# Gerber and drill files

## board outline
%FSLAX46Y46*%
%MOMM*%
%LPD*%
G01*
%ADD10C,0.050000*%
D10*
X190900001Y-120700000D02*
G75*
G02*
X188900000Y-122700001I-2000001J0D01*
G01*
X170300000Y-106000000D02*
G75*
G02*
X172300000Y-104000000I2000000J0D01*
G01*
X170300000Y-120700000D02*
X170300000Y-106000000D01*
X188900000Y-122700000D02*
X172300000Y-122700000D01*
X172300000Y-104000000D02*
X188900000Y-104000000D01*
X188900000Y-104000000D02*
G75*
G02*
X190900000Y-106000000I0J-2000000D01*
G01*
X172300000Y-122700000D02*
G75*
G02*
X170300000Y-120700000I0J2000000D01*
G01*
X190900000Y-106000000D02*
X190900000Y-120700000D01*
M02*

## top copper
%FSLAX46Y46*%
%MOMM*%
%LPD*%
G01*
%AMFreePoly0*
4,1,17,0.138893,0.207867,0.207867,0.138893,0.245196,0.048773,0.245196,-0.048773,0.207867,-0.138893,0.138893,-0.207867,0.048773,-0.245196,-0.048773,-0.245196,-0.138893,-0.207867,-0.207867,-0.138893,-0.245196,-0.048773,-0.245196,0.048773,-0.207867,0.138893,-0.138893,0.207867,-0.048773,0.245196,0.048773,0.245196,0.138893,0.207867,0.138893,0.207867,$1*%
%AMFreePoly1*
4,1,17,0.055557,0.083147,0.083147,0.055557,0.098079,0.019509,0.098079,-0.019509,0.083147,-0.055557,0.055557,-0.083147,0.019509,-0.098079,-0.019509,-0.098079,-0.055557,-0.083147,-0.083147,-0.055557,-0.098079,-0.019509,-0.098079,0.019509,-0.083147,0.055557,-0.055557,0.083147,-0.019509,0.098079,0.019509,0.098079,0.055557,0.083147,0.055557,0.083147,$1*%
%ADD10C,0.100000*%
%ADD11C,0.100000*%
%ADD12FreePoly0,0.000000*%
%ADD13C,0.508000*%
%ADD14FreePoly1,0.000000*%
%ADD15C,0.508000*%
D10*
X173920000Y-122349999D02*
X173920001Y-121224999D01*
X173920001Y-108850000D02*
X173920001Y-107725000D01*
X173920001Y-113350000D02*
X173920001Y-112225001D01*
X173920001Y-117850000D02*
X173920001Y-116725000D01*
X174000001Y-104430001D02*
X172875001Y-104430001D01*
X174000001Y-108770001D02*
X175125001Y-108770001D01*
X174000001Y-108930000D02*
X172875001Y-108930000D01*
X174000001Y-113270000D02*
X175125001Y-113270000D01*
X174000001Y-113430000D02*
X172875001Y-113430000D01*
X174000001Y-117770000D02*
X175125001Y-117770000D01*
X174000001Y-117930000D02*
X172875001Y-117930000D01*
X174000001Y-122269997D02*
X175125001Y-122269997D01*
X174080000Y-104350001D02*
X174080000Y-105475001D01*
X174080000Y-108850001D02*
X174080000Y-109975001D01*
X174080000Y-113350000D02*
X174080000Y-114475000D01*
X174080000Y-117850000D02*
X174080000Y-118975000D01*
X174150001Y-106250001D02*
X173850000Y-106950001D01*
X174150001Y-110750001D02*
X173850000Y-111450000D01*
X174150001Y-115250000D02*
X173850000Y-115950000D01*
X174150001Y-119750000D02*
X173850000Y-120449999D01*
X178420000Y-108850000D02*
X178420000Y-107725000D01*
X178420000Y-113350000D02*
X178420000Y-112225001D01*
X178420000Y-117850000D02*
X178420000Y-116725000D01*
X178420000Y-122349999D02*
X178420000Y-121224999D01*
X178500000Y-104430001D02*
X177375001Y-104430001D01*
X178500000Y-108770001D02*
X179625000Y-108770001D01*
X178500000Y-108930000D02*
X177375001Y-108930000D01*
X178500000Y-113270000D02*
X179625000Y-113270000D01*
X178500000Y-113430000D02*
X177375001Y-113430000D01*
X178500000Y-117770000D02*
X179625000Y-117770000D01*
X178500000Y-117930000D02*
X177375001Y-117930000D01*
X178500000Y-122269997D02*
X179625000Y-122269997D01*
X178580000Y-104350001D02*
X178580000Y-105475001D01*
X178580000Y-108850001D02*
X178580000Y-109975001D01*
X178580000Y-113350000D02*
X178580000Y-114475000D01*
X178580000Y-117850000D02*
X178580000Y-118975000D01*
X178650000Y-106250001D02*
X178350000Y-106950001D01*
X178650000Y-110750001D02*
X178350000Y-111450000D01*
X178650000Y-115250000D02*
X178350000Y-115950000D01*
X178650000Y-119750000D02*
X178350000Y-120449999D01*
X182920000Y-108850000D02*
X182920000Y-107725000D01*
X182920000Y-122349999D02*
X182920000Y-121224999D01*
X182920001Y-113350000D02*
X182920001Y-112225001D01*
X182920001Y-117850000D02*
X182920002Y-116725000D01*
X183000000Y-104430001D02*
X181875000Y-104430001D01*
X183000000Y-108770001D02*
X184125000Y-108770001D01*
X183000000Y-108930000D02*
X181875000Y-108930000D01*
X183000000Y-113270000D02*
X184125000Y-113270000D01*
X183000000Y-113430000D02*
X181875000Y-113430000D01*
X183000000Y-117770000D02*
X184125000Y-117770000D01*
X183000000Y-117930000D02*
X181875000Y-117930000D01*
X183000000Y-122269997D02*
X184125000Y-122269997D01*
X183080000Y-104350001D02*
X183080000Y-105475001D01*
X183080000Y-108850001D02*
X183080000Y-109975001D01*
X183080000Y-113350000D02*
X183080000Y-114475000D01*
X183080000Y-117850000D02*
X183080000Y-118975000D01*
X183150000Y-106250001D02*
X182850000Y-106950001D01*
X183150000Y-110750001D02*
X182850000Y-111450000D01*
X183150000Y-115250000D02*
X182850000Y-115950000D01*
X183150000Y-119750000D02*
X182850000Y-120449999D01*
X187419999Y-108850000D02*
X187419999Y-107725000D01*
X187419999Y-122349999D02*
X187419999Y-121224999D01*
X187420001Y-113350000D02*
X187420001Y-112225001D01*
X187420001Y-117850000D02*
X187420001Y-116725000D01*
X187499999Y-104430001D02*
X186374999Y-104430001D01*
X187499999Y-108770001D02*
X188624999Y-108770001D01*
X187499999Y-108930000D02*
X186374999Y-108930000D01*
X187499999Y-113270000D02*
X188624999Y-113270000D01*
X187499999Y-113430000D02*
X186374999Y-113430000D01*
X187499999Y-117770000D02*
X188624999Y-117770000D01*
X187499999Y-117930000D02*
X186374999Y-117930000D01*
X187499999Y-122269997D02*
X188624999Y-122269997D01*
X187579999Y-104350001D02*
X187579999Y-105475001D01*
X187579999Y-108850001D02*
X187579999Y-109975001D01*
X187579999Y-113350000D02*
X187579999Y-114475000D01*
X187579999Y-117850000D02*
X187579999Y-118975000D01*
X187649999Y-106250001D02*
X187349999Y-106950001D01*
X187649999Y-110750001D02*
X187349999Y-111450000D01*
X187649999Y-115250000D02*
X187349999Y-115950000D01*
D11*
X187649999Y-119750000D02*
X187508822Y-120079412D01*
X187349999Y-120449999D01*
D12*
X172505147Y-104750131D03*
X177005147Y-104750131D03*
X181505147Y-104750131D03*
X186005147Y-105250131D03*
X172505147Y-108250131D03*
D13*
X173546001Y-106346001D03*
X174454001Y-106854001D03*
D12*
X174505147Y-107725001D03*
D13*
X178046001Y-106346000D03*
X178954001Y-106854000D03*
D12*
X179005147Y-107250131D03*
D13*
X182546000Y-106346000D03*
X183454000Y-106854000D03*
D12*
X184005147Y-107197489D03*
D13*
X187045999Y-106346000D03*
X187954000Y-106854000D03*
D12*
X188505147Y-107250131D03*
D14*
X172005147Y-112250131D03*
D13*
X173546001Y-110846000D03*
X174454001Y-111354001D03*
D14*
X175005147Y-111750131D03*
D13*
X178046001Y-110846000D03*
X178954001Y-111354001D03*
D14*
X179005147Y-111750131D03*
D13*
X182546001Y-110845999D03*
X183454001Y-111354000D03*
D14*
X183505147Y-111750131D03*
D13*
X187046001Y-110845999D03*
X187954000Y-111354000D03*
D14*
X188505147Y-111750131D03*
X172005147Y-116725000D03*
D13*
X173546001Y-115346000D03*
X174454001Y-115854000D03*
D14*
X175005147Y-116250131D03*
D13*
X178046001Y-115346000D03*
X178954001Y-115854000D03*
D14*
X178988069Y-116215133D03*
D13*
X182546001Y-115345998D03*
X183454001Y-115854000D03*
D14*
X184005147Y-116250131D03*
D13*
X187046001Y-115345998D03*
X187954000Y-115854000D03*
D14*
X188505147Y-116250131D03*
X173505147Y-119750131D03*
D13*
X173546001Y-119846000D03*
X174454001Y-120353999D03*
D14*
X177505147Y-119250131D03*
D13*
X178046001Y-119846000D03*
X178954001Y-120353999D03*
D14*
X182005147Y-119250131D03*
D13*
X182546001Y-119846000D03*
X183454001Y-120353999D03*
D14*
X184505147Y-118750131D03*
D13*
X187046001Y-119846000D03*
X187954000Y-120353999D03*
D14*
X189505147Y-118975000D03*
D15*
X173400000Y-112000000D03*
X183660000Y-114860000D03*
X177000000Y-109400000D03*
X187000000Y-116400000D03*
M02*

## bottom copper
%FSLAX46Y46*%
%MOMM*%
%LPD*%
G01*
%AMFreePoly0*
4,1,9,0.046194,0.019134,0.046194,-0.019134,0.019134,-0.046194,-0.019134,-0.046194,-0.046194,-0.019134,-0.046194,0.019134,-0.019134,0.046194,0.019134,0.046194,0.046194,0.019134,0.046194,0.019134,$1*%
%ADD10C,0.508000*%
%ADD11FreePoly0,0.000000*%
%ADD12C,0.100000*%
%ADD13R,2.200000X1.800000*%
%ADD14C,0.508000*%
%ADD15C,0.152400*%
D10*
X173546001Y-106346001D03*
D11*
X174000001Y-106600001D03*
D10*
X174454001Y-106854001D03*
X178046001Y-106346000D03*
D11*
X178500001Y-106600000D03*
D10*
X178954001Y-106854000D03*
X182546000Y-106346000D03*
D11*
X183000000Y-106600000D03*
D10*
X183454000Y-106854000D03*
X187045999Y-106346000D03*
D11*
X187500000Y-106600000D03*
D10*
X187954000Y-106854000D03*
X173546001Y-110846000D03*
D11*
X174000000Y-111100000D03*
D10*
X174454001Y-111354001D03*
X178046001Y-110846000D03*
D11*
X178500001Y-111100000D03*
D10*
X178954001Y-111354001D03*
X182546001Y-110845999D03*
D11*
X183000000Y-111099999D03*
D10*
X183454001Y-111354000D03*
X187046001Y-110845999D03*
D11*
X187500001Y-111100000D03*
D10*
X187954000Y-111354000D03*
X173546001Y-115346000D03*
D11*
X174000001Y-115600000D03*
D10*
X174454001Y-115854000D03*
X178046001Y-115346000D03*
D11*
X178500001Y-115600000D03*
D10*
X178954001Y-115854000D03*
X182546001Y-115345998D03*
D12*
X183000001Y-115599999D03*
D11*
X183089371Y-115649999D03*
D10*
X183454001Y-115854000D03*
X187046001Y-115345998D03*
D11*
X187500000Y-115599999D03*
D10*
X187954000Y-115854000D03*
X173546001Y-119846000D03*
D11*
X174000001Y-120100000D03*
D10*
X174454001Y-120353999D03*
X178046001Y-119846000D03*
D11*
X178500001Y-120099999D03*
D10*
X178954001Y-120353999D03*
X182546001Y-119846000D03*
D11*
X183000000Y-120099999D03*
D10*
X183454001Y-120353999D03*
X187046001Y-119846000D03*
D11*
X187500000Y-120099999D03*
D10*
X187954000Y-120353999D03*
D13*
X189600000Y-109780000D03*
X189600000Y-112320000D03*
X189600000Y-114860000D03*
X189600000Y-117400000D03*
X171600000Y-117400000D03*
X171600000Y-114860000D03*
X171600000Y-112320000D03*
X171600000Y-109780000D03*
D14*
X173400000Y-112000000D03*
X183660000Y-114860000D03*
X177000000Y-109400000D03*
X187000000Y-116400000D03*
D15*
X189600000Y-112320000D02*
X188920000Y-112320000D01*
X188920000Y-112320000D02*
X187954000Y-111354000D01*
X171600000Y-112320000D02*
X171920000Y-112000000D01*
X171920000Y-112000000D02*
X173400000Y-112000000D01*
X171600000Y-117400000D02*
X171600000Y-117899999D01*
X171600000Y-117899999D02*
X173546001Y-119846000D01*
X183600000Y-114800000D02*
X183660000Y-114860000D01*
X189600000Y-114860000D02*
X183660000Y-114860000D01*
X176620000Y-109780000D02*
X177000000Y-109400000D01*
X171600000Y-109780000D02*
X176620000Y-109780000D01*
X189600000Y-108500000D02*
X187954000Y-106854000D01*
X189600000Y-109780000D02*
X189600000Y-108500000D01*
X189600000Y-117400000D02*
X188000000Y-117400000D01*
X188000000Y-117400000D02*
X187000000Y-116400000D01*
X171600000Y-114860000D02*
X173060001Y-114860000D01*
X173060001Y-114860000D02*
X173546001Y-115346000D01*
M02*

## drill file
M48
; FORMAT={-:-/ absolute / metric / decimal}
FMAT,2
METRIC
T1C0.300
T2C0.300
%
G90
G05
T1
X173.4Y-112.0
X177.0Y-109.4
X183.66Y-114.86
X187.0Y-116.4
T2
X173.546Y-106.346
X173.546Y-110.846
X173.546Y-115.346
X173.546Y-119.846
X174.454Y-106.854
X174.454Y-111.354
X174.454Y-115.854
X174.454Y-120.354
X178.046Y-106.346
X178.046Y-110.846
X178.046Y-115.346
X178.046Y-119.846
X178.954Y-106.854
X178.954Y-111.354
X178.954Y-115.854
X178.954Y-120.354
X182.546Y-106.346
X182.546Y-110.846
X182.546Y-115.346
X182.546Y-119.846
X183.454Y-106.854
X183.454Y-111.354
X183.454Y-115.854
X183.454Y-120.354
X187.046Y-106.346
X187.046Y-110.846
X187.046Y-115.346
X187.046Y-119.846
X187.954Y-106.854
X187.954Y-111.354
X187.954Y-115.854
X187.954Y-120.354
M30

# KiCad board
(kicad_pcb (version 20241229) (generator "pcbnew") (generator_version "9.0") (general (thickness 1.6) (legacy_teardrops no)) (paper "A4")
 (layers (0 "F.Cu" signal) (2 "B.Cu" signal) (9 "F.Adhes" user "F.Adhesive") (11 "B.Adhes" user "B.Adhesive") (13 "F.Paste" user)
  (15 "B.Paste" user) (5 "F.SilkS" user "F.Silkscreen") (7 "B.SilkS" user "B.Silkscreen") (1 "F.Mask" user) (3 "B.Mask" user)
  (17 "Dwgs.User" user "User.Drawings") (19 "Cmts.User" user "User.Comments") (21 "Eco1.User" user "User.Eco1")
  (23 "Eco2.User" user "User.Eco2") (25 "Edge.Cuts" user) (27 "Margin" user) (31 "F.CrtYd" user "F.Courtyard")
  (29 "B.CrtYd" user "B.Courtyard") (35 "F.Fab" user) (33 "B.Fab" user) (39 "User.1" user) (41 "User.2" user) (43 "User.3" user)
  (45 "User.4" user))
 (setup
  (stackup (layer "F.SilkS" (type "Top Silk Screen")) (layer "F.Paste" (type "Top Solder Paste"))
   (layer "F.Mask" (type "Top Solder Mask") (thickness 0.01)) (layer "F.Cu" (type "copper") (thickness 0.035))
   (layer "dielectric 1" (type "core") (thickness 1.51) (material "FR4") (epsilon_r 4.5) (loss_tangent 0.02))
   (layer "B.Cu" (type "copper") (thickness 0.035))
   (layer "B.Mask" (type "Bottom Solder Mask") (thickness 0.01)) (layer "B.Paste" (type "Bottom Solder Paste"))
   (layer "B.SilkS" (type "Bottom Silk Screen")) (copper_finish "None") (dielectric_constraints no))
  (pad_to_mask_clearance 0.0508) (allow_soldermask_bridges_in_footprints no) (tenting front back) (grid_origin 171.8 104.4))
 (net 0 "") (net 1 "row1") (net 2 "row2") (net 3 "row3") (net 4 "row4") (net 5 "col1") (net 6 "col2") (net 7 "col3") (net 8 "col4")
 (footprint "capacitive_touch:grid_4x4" (layer "F.Cu") (at 180.505147 124.750131)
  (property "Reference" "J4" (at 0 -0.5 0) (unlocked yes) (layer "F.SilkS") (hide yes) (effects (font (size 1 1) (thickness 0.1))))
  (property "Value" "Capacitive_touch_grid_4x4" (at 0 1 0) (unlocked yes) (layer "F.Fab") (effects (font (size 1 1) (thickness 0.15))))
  (fp_line (start -6.585147 -2.400132) (end -6.585146 -3.525132) (stroke (width 0.1) (type solid)) (layer "F.Cu"))
  (fp_line (start -6.585146 -15.900131) (end -6.585146 -17.025131) (stroke (width 0.1) (type solid)) (layer "F.Cu"))
  (fp_line (start -6.585146 -11.400131) (end -6.585146 -12.52513) (stroke (width 0.1) (type solid)) (layer "F.Cu"))
  (fp_line (start -6.585146 -6.900131) (end -6.585146 -8.025131) (stroke (width 0.1) (type solid)) (layer "F.Cu"))
  (fp_line (start -6.505146 -20.32013) (end -7.630146 -20.32013) (stroke (width 0.1) (type solid)) (layer "F.Cu"))
  (fp_line (start -6.505146 -15.98013) (end -5.380146 -15.98013) (stroke (width 0.1) (type solid)) (layer "F.Cu"))
  (fp_line (start -6.505146 -15.820131) (end -7.630146 -15.820131) (stroke (width 0.1) (type solid)) (layer "F.Cu"))
  (fp_line (start -6.505146 -11.480131) (end -5.380146 -11.480131) (stroke (width 0.1) (type solid)) (layer "F.Cu"))
  (fp_line (start -6.505146 -11.320131) (end -7.630146 -11.320131) (stroke (width 0.1) (type solid)) (layer "F.Cu"))
  (fp_line (start -6.505146 -6.980131) (end -5.380146 -6.980131) (stroke (width 0.1) (type solid)) (layer "F.Cu"))
  (fp_line (start -6.505146 -6.820131) (end -7.630146 -6.820131) (stroke (width 0.1) (type solid)) (layer "F.Cu"))
  (fp_line (start -6.505146 -2.480134) (end -5.380146 -2.480134) (stroke (width 0.1) (type solid)) (layer "F.Cu"))
  (fp_line (start -6.425147 -20.40013) (end -6.425147 -19.27513) (stroke (width 0.1) (type solid)) (layer "F.Cu"))
  (fp_line (start -6.425147 -15.90013) (end -6.425147 -14.77513) (stroke (width 0.1) (type solid)) (layer "F.Cu"))
  (fp_line (start -6.425147 -11.400131) (end -6.425147 -10.275131) (stroke (width 0.1) (type solid)) (layer "F.Cu"))
  (fp_line (start -6.425147 -6.900131) (end -6.425147 -5.775131) (stroke (width 0.1) (type solid)) (layer "F.Cu"))
  (fp_line (start -6.355146 -18.50013) (end -6.655147 -17.80013) (stroke (width 0.1) (type solid)) (layer "F.Cu"))
  (fp_line (start -6.355146 -14.00013) (end -6.655147 -13.300131) (stroke (width 0.1) (type solid)) (layer "F.Cu"))
  (fp_line (start -6.355146 -9.500131) (end -6.655147 -8.800131) (stroke (width 0.1) (type solid)) (layer "F.Cu"))
  (fp_line (start -6.355146 -5.000131) (end -6.655147 -4.300132) (stroke (width 0.1) (type solid)) (layer "F.Cu"))
  (fp_line (start -2.085147 -15.900131) (end -2.085147 -17.025131) (stroke (width 0.1) (type solid)) (layer "F.Cu"))
  (fp_line (start -2.085147 -11.400131) (end -2.085147 -12.52513) (stroke (width 0.1) (type solid)) (layer "F.Cu"))
  (fp_line (start -2.085147 -6.900131) (end -2.085147 -8.025131) (stroke (width 0.1) (type solid)) (layer "F.Cu"))
  (fp_line (start -2.085147 -2.400132) (end -2.085147 -3.525132) (stroke (width 0.1) (type solid)) (layer "F.Cu"))
  (fp_line (start -2.005147 -20.32013) (end -3.130146 -20.32013) (stroke (width 0.1) (type solid)) (layer "F.Cu"))
  (fp_line (start -2.005147 -15.98013) (end -0.880147 -15.98013) (stroke (width 0.1) (type solid)) (layer "F.Cu"))
  (fp_line (start -2.005147 -15.820131) (end -3.130146 -15.820131) (stroke (width 0.1) (type solid)) (layer "F.Cu"))
  (fp_line (start -2.005147 -11.480131) (end -0.880147 -11.480131) (stroke (width 0.1) (type solid)) (layer "F.Cu"))
  (fp_line (start -2.005147 -11.320131) (end -3.130146 -11.320131) (stroke (width 0.1) (type solid)) (layer "F.Cu"))
  (fp_line (start -2.005147 -6.980131) (end -0.880147 -6.980131) (stroke (width 0.1) (type solid)) (layer "F.Cu"))
  (fp_line (start -2.005147 -6.820131) (end -3.130146 -6.820131) (stroke (width 0.1) (type solid)) (layer "F.Cu"))
  (fp_line (start -2.005147 -2.480134) (end -0.880147 -2.480134) (stroke (width 0.1) (type solid)) (layer "F.Cu"))
  (fp_line (start -1.925147 -20.40013) (end -1.925147 -19.27513) (stroke (width 0.1) (type solid)) (layer "F.Cu"))
  (fp_line (start -1.925147 -15.90013) (end -1.925147 -14.77513) (stroke (width 0.1) (type solid)) (layer "F.Cu"))
  (fp_line (start -1.925147 -11.400131) (end -1.925147 -10.275131) (stroke (width 0.1) (type solid)) (layer "F.Cu"))
  (fp_line (start -1.925147 -6.900131) (end -1.925147 -5.775131) (stroke (width 0.1) (type solid)) (layer "F.Cu"))
  (fp_line (start -1.855147 -18.50013) (end -2.155147 -17.80013) (stroke (width 0.1) (type solid)) (layer "F.Cu"))
  (fp_line (start -1.855147 -14.00013) (end -2.155147 -13.300131) (stroke (width 0.1) (type solid)) (layer "F.Cu"))
  (fp_line (start -1.855147 -9.500131) (end -2.155147 -8.800131) (stroke (width 0.1) (type solid)) (layer "F.Cu"))
  (fp_line (start -1.855147 -5.000131) (end -2.155147 -4.300132) (stroke (width 0.1) (type solid)) (layer "F.Cu"))
  (fp_line (start 2.414853 -15.900131) (end 2.414853 -17.025131) (stroke (width 0.1) (type solid)) (layer "F.Cu"))
  (fp_line (start 2.414853 -2.400132) (end 2.414853 -3.525132) (stroke (width 0.1) (type solid)) (layer "F.Cu"))
  (fp_line (start 2.414854 -11.400131) (end 2.414854 -12.52513) (stroke (width 0.1) (type solid)) (layer "F.Cu"))
  (fp_line (start 2.414854 -6.900131) (end 2.414855 -8.025131) (stroke (width 0.1) (type solid)) (layer "F.Cu"))
  (fp_line (start 2.494853 -20.32013) (end 1.369853 -20.32013) (stroke (width 0.1) (type solid)) (layer "F.Cu"))
  (fp_line (start 2.494853 -15.98013) (end 3.619853 -15.98013) (stroke (width 0.1) (type solid)) (layer "F.Cu"))
  (fp_line (start 2.494853 -15.820131) (end 1.369853 -15.820131) (stroke (width 0.1) (type solid)) (layer "F.Cu"))
  (fp_line (start 2.494853 -11.480131) (end 3.619853 -11.480131) (stroke (width 0.1) (type solid)) (layer "F.Cu"))
  (fp_line (start 2.494853 -11.320131) (end 1.369853 -11.320131) (stroke (width 0.1) (type solid)) (layer "F.Cu"))
  (fp_line (start 2.494853 -6.980131) (end 3.619853 -6.980131) (stroke (width 0.1) (type solid)) (layer "F.Cu"))
  (fp_line (start 2.494853 -6.820131) (end 1.369853 -6.820131) (stroke (width 0.1) (type solid)) (layer "F.Cu"))
  (fp_line (start 2.494853 -2.480134) (end 3.619853 -2.480134) (stroke (width 0.1) (type solid)) (layer "F.Cu"))
  (fp_line (start 2.574853 -20.40013) (end 2.574853 -19.27513) (stroke (width 0.1) (type solid)) (layer "F.Cu"))
  (fp_line (start 2.574853 -15.90013) (end 2.574853 -14.77513) (stroke (width 0.1) (type solid)) (layer "F.Cu"))
  (fp_line (start 2.574853 -11.400131) (end 2.574853 -10.275131) (stroke (width 0.1) (type solid)) (layer "F.Cu"))
  (fp_line (start 2.574853 -6.900131) (end 2.574853 -5.775131) (stroke (width 0.1) (type solid)) (layer "F.Cu"))
  (fp_line (start 2.644853 -18.50013) (end 2.344853 -17.80013) (stroke (width 0.1) (type solid)) (layer "F.Cu"))
  (fp_line (start 2.644853 -14.00013) (end 2.344853 -13.300131) (stroke (width 0.1) (type solid)) (layer "F.Cu"))
  (fp_line (start 2.644853 -9.500131) (end 2.344853 -8.800131) (stroke (width 0.1) (type solid)) (layer "F.Cu"))
  (fp_line (start 2.644853 -5.000131) (end 2.344853 -4.300132) (stroke (width 0.1) (type solid)) (layer "F.Cu"))
  (fp_line (start 6.914852 -15.900131) (end 6.914852 -17.025131) (stroke (width 0.1) (type solid)) (layer "F.Cu"))
  (fp_line (start 6.914852 -2.400132) (end 6.914852 -3.525132) (stroke (width 0.1) (type solid)) (layer "F.Cu"))
  (fp_line (start 6.914854 -11.400131) (end 6.914854 -12.52513) (stroke (width 0.1) (type solid)) (layer "F.Cu"))
  (fp_line (start 6.914854 -6.900131) (end 6.914854 -8.025131) (stroke (width 0.1) (type solid)) (layer "F.Cu"))
  (fp_line (start 6.994852 -20.32013) (end 5.869852 -20.32013) (stroke (width 0.1) (type solid)) (layer "F.Cu"))
  (fp_line (start 6.994852 -15.98013) (end 8.119852 -15.98013) (stroke (width 0.1) (type solid)) (layer "F.Cu"))
  (fp_line (start 6.994852 -15.820131) (end 5.869852 -15.820131) (stroke (width 0.1) (type solid)) (layer "F.Cu"))
  (fp_line (start 6.994852 -11.480131) (end 8.119852 -11.480131) (stroke (width 0.1) (type solid)) (layer "F.Cu"))
  (fp_line (start 6.994852 -11.320131) (end 5.869852 -11.320131) (stroke (width 0.1) (type solid)) (layer "F.Cu"))
  (fp_line (start 6.994852 -6.980131) (end 8.119852 -6.980131) (stroke (width 0.1) (type solid)) (layer "F.Cu"))
  (fp_line (start 6.994852 -6.820131) (end 5.869852 -6.820131) (stroke (width 0.1) (type solid)) (layer "F.Cu"))
  (fp_line (start 6.994852 -2.480134) (end 8.119852 -2.480134) (stroke (width 0.1) (type solid)) (layer "F.Cu"))
  (fp_line (start 7.074852 -20.40013) (end 7.074852 -19.27513) (stroke (width 0.1) (type solid)) (layer "F.Cu"))
  (fp_line (start 7.074852 -15.90013) (end 7.074852 -14.77513) (stroke (width 0.1) (type solid)) (layer "F.Cu"))
  (fp_line (start 7.074852 -11.400131) (end 7.074852 -10.275131) (stroke (width 0.1) (type solid)) (layer "F.Cu"))
  (fp_line (start 7.074852 -6.900131) (end 7.074852 -5.775131) (stroke (width 0.1) (type solid)) (layer "F.Cu"))
  (fp_line (start 7.144852 -18.50013) (end 6.844852 -17.80013) (stroke (width 0.1) (type solid)) (layer "F.Cu"))
  (fp_line (start 7.144852 -14.00013) (end 6.844852 -13.300131) (stroke (width 0.1) (type solid)) (layer "F.Cu"))
  (fp_line (start 7.144852 -9.500131) (end 6.844852 -8.800131) (stroke (width 0.1) (type solid)) (layer "F.Cu"))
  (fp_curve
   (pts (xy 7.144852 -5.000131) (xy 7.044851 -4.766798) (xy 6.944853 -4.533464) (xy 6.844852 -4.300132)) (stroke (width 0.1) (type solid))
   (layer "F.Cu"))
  (pad "1" smd custom (at -8 -20) (size 0.5 0.5) (layers "F.Cu") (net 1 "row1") (options (clearance outline) (anchor circle)) (primitives))
  (pad "2" smd custom (at -3.5 -20) (size 0.5 0.5) (layers "F.Cu") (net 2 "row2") (options (clearance outline) (anchor circle)) (primitives))
  (pad "3" smd custom (at 1 -20) (size 0.5 0.5) (layers "F.Cu") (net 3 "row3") (options (clearance outline) (anchor circle)) (primitives))
  (pad "4" smd custom (at 5.5 -19.5) (size 0.5 0.5) (layers "F.Cu") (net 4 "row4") (options (clearance outline) (anchor circle))
   (primitives))
  (pad "5" smd custom (at -8 -16.5) (size 0.5 0.5) (layers "F.Cu") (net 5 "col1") (options (clearance outline) (anchor circle)) (primitives))
  (pad "5" thru_hole circle (at -6.959146 -18.40413) (size 0.508 0.508) (drill 0.3) (layers "*.Cu") (remove_unused_layers no) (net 5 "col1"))
  (pad "5" smd custom (at -6.505146 -18.15013) (size 0.1 0.1) (layers "B.Cu") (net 5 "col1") (options (clearance outline) (anchor circle))
   (primitives))
  (pad "5" thru_hole circle (at -6.051146 -17.89613) (size 0.508 0.508) (drill 0.3) (layers "*.Cu") (remove_unused_layers no) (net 5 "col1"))
  (pad "5" smd custom (at -6 -17.02513) (size 0.5 0.5) (layers "F.Cu") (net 5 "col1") (options (clearance outline) (anchor circle))
   (primitives))
  (pad "5" thru_hole circle (at -2.459146 -18.404131) (size 0.508 0.508) (drill 0.3) (layers "*.Cu") (remove_unused_layers no)
   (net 5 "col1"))
  (pad "5" smd custom (at -2.005146 -18.150131) (size 0.1 0.1) (layers "B.Cu") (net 5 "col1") (options (clearance outline) (anchor circle))
   (primitives))
  (pad "5" thru_hole circle (at -1.551146 -17.896131) (size 0.508 0.508) (drill 0.3) (layers "*.Cu") (remove_unused_layers no)
   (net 5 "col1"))
  (pad "5" smd custom (at -1.5 -17.5) (size 0.5 0.5) (layers "F.Cu") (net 5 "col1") (options (clearance outline) (anchor circle))
   (primitives))
  (pad "5" thru_hole circle (at 2.040853 -18.404131) (size 0.508 0.508) (drill 0.3) (layers "*.Cu") (remove_unused_layers no) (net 5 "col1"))
  (pad "5" smd custom (at 2.494853 -18.150131) (size 0.1 0.1) (layers "B.Cu") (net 5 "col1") (options (clearance outline) (anchor circle))
   (primitives))
  (pad "5" thru_hole circle (at 2.948853 -17.896131) (size 0.508 0.508) (drill 0.3) (layers "*.Cu") (remove_unused_layers no) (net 5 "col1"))
  (pad "5" smd custom (at 3.5 -17.552642) (size 0.5 0.5) (layers "F.Cu") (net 5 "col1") (options (clearance outline) (anchor circle))
   (primitives))
  (pad "5" thru_hole circle (at 6.540852 -18.404131) (size 0.508 0.508) (drill 0.3) (layers "*.Cu") (remove_unused_layers no) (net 5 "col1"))
  (pad "5" smd custom (at 6.994853 -18.150131) (size 0.1 0.1) (layers "B.Cu") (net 5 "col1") (options (clearance outline) (anchor circle))
   (primitives))
  (pad "5" thru_hole circle (at 7.448853 -17.896131) (size 0.508 0.508) (drill 0.3) (layers "*.Cu") (remove_unused_layers no) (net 5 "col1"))
  (pad "5" smd custom (at 8 -17.5) (size 0.5 0.5) (layers "F.Cu") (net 5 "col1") (options (clearance outline) (anchor circle)) (primitives))
  (pad "6" smd custom (at -8.5 -12.5) (size 0.2 0.2) (layers "F.Cu") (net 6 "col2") (options (clearance outline) (anchor circle))
   (primitives))
  (pad "6" thru_hole circle (at -6.959146 -13.904131) (size 0.508 0.508) (drill 0.3) (layers "*.Cu") (remove_unused_layers no)
   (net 6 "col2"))
  (pad "6" smd custom (at -6.505147 -13.650131) (size 0.1 0.1) (layers "B.Cu") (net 6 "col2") (options (clearance outline) (anchor circle))
   (primitives))
  (pad "6" thru_hole circle (at -6.051146 -13.39613) (size 0.508 0.508) (drill 0.3) (layers "*.Cu") (remove_unused_layers no) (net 6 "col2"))
  (pad "6" smd custom (at -5.5 -13) (size 0.2 0.2) (layers "F.Cu") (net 6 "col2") (options (clearance outline) (anchor circle)) (primitives))
  (pad "6" thru_hole circle (at -2.459146 -13.904131) (size 0.508 0.508) (drill 0.3) (layers "*.Cu") (remove_unused_layers no)
   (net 6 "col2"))
  (pad "6" smd custom (at -2.005146 -13.650131) (size 0.1 0.1) (layers "B.Cu") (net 6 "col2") (options (clearance outline) (anchor circle))
   (primitives))
  (pad "6" thru_hole circle (at -1.551146 -13.39613) (size 0.508 0.508) (drill 0.3) (layers "*.Cu") (remove_unused_layers no) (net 6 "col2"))
  (pad "6" smd custom (at -1.5 -13) (size 0.2 0.2) (layers "F.Cu") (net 6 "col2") (options (clearance outline) (anchor circle)) (primitives))
  (pad "6" thru_hole circle (at 2.040854 -13.904132) (size 0.508 0.508) (drill 0.3) (layers "*.Cu") (remove_unused_layers no) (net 6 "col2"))
  (pad "6" smd custom (at 2.494853 -13.650132) (size 0.1 0.1) (layers "B.Cu") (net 6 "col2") (options (clearance outline) (anchor circle))
   (primitives))
  (pad "6" thru_hole circle (at 2.948854 -13.396131) (size 0.508 0.508) (drill 0.3) (layers "*.Cu") (remove_unused_layers no) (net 6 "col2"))
  (pad "6" smd custom (at 3 -13) (size 0.2 0.2) (layers "F.Cu") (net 6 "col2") (options (clearance outline) (anchor circle)) (primitives))
  (pad "6" thru_hole circle (at 6.540854 -13.904132) (size 0.508 0.508) (drill 0.3) (layers "*.Cu") (remove_unused_layers no) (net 6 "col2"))
  (pad "6" smd custom (at 6.994854 -13.650131) (size 0.1 0.1) (layers "B.Cu") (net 6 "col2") (options (clearance outline) (anchor circle))
   (primitives))
  (pad "6" thru_hole circle (at 7.448853 -13.396131) (size 0.508 0.508) (drill 0.3) (layers "*.Cu") (remove_unused_layers no) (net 6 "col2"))
  (pad "6" smd custom (at 8 -13) (size 0.2 0.2) (layers "F.Cu") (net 6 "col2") (options (clearance outline) (anchor circle)) (primitives))
  (pad "7" smd custom (at -8.5 -8.025131) (size 0.2 0.2) (layers "F.Cu") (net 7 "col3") (options (clearance outline) (anchor circle))
   (primitives))
  (pad "7" thru_hole circle (at -6.959146 -9.404131) (size 0.508 0.508) (drill 0.3) (layers "*.Cu") (remove_unused_layers no) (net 7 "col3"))
  (pad "7" smd custom (at -6.505146 -9.150131) (size 0.1 0.1) (layers "B.Cu") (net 7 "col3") (options (clearance outline) (anchor circle))
   (primitives))
  (pad "7" thru_hole circle (at -6.051146 -8.896131) (size 0.508 0.508) (drill 0.3) (layers "*.Cu") (remove_unused_layers no) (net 7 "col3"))
  (pad "7" smd custom (at -5.5 -8.5) (size 0.2 0.2) (layers "F.Cu") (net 7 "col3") (options (clearance outline) (anchor circle))
   (primitives))
  (pad "7" thru_hole circle (at -2.459146 -9.404131) (size 0.508 0.508) (drill 0.3) (layers "*.Cu") (remove_unused_layers no) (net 7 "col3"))
  (pad "7" smd custom (at -2.005146 -9.150131) (size 0.1 0.1) (layers "B.Cu") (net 7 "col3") (options (clearance outline) (anchor circle))
   (primitives))
  (pad "7" thru_hole circle (at -1.551146 -8.896131) (size 0.508 0.508) (drill 0.3) (layers "*.Cu") (remove_unused_layers no) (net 7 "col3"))
  (pad "7" smd custom (at -1.517078 -8.534998) (size 0.2 0.2) (layers "F.Cu") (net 7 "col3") (options (clearance outline) (anchor circle))
   (primitives))
  (pad "7" thru_hole circle (at 2.040854 -9.404133) (size 0.508 0.508) (drill 0.3) (layers "*.Cu") (remove_unused_layers no) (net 7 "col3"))
  (pad "7" smd circle (at 2.494854 -9.150132) (size 0.1 0.1) (layers "B.Cu") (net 7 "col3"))
  (pad "7" smd custom (at 2.584224 -9.100132) (size 0.1 0.1) (layers "B.Cu") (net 7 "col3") (options (clearance outline) (anchor circle))
   (primitives))
  (pad "7" thru_hole circle (at 2.948854 -8.896131) (size 0.508 0.508) (drill 0.3) (layers "*.Cu") (remove_unused_layers no) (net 7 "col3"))
  (pad "7" smd custom (at 3.5 -8.5) (size 0.2 0.2) (layers "F.Cu") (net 7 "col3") (options (clearance outline) (anchor circle)) (primitives))
  (pad "7" thru_hole circle (at 6.540854 -9.404133) (size 0.508 0.508) (drill 0.3) (layers "*.Cu") (remove_unused_layers no) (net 7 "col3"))
  (pad "7" smd custom (at 6.994853 -9.150132) (size 0.1 0.1) (layers "B.Cu") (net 7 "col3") (options (clearance outline) (anchor circle))
   (primitives))
  (pad "7" thru_hole circle (at 7.448853 -8.896131) (size 0.508 0.508) (drill 0.3) (layers "*.Cu") (remove_unused_layers no) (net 7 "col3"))
  (pad "7" smd custom (at 8 -8.5) (size 0.2 0.2) (layers "F.Cu") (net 7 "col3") (options (clearance outline) (anchor circle)) (primitives))
  (pad "8" smd custom (at -7 -5) (size 0.2 0.2) (layers "F.Cu") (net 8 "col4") (options (clearance outline) (anchor circle)) (primitives))
  (pad "8" thru_hole circle (at -6.959146 -4.904131) (size 0.508 0.508) (drill 0.3) (layers "*.Cu") (remove_unused_layers no) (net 8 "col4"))
  (pad "8" smd custom (at -6.505146 -4.650131) (size 0.1 0.1) (layers "B.Cu") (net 8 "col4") (options (clearance outline) (anchor circle))
   (primitives))
  (pad "8" thru_hole circle (at -6.051146 -4.396132) (size 0.508 0.508) (drill 0.3) (layers "*.Cu") (remove_unused_layers no) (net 8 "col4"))
  (pad "8" smd custom (at -3 -5.5) (size 0.2 0.2) (layers "F.Cu") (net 8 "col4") (options (clearance outline) (anchor circle)) (primitives))
  (pad "8" thru_hole circle (at -2.459146 -4.904131) (size 0.508 0.508) (drill 0.3) (layers "*.Cu") (remove_unused_layers no) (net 8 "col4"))
  (pad "8" smd custom (at -2.005146 -4.650132) (size 0.1 0.1) (layers "B.Cu") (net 8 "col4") (options (clearance outline) (anchor circle))
   (primitives))
  (pad "8" thru_hole circle (at -1.551146 -4.396132) (size 0.508 0.508) (drill 0.3) (layers "*.Cu") (remove_unused_layers no) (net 8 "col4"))
  (pad "8" smd custom (at 1.5 -5.5) (size 0.2 0.2) (layers "F.Cu") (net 8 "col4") (options (clearance outline) (anchor circle)) (primitives))
  (pad "8" thru_hole circle (at 2.040854 -4.904131) (size 0.508 0.508) (drill 0.3) (layers "*.Cu") (remove_unused_layers no) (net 8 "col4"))
  (pad "8" smd custom (at 2.494853 -4.650132) (size 0.1 0.1) (layers "B.Cu") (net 8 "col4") (options (clearance outline) (anchor circle))
   (primitives))
  (pad "8" thru_hole circle (at 2.948854 -4.396132) (size 0.508 0.508) (drill 0.3) (layers "*.Cu") (remove_unused_layers no) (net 8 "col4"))
  (pad "8" smd custom (at 4 -6) (size 0.2 0.2) (layers "F.Cu") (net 8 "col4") (options (clearance outline) (anchor circle)) (primitives))
  (pad "8" thru_hole circle (at 6.540854 -4.904131) (size 0.508 0.508) (drill 0.3) (layers "*.Cu") (remove_unused_layers no) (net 8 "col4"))
  (pad "8" smd custom (at 6.994853 -4.650132) (size 0.1 0.1) (layers "B.Cu") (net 8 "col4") (options (clearance outline) (anchor circle))
   (primitives))
  (pad "8" thru_hole circle (at 7.448853 -4.396132) (size 0.508 0.508) (drill 0.3) (layers "*.Cu") (remove_unused_layers no) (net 8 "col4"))
  (pad "8" smd custom (at 9 -5.775131) (size 0.2 0.2) (layers "F.Cu") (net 8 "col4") (options (clearance outline) (anchor circle))
   (primitives)))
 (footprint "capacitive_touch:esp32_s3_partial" (layer "B.Cu") (at 180.6 113.59 -90)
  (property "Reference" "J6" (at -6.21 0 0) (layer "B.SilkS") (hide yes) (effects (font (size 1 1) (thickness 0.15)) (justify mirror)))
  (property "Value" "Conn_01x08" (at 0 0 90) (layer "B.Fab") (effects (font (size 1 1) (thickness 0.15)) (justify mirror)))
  (pad "1" smd rect (at -3.81 -9 270) (size 1.8 2.2) (layers "B.Cu" "B.Mask" "B.Paste") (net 5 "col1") (thermal_bridge_angle 45))
  (pad "2" smd rect (at -1.27 -9 270) (size 1.8 2.2) (layers "B.Cu" "B.Mask" "B.Paste") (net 6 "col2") (thermal_bridge_angle 45))
  (pad "3" smd rect (at 1.27 -9 270) (size 1.8 2.2) (layers "B.Cu" "B.Mask" "B.Paste") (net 3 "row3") (thermal_bridge_angle 45))
  (pad "4" smd rect (at 3.81 -9 270) (size 1.8 2.2) (layers "B.Cu" "B.Mask" "B.Paste") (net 4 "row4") (thermal_bridge_angle 45))
  (pad "5" smd rect (at 3.81 9 270) (size 1.8 2.2) (layers "B.Cu" "B.Mask" "B.Paste") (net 8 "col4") (thermal_bridge_angle 45))
  (pad "6" smd rect (at 1.27 9 270) (size 1.8 2.2) (layers "B.Cu" "B.Mask" "B.Paste") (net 7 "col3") (thermal_bridge_angle 45))
  (pad "7" smd rect (at -1.27 9 270) (size 1.8 2.2) (layers "B.Cu" "B.Mask" "B.Paste") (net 1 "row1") (thermal_bridge_angle 45))
  (pad "8" smd rect (at -3.81 9 270) (size 1.8 2.2) (layers "B.Cu" "B.Mask" "B.Paste") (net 2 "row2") (thermal_bridge_angle 45)))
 (gr_arc (start 190.900001 120.7) (mid 190.314214 122.114214) (end 188.9 122.700001) (stroke (width 0.05) (type default))
  (layer "Edge.Cuts"))
 (gr_arc (start 170.3 106) (mid 170.885786 104.585786) (end 172.3 104) (stroke (width 0.05) (type default)) (layer "Edge.Cuts"))
 (gr_line (start 170.3 120.7) (end 170.3 106) (stroke (width 0.05) (type default)) (layer "Edge.Cuts"))
 (gr_line (start 188.9 122.7) (end 172.3 122.7) (stroke (width 0.05) (type default)) (layer "Edge.Cuts"))
 (gr_line (start 172.3 104) (end 188.9 104) (stroke (width 0.05) (type default)) (layer "Edge.Cuts"))
 (gr_arc (start 188.9 104) (mid 190.314214 104.585786) (end 190.9 106) (stroke (width 0.05) (type default)) (layer "Edge.Cuts"))
 (gr_arc (start 172.3 122.7) (mid 170.885786 122.114214) (end 170.3 120.7) (stroke (width 0.05) (type default)) (layer "Edge.Cuts"))
 (gr_line (start 190.9 106) (end 190.9 120.7) (stroke (width 0.05) (type default)) (layer "Edge.Cuts"))
 (segment (start 189.6 112.32) (end 188.92 112.32) (width 0.1524) (layer "B.Cu") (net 6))
 (segment (start 188.92 112.32) (end 187.954 111.354) (width 0.1524) (layer "B.Cu") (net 6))
 (via (at 173.4 112) (size 0.508) (drill 0.3) (layers "F.Cu" "B.Cu") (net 1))
 (segment (start 171.6 112.32) (end 171.92 112) (width 0.1524) (layer "B.Cu") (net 1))
 (segment (start 171.92 112) (end 173.4 112) (width 0.1524) (layer "B.Cu") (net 1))
 (segment (start 171.6 117.4) (end 171.6 117.899999) (width 0.1524) (layer "B.Cu") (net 8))
 (segment (start 171.6 117.899999) (end 173.546001 119.846) (width 0.1524) (layer "B.Cu") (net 8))
 (via (at 183.66 114.86) (size 0.508) (drill 0.3) (layers "F.Cu" "B.Cu") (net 3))
 (segment (start 183.6 114.8) (end 183.66 114.86) (width 0.1524) (layer "B.Cu") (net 3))
 (segment (start 189.6 114.86) (end 183.66 114.86) (width 0.1524) (layer "B.Cu") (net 3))
 (via (at 177 109.4) (size 0.508) (drill 0.3) (layers "F.Cu" "B.Cu") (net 2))
 (segment (start 176.62 109.78) (end 177 109.4) (width 0.1524) (layer "B.Cu") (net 2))
 (segment (start 171.6 109.78) (end 176.62 109.78) (width 0.1524) (layer "B.Cu") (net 2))
 (segment (start 189.6 108.5) (end 187.954 106.854) (width 0.1524) (layer "B.Cu") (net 5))
 (segment (start 189.6 109.78) (end 189.6 108.5) (width 0.1524) (layer "B.Cu") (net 5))
 (via (at 187 116.4) (size 0.508) (drill 0.3) (layers "F.Cu" "B.Cu") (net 4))
 (segment (start 189.6 117.4) (end 188 117.4) (width 0.1524) (layer "B.Cu") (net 4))
 (segment (start 188 117.4) (end 187 116.4) (width 0.1524) (layer "B.Cu") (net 4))
 (segment (start 171.6 114.86) (end 173.060001 114.86) (width 0.1524) (layer "B.Cu") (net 7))
 (segment (start 173.060001 114.86) (end 173.546001 115.346) (width 0.1524) (layer "B.Cu") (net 7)))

